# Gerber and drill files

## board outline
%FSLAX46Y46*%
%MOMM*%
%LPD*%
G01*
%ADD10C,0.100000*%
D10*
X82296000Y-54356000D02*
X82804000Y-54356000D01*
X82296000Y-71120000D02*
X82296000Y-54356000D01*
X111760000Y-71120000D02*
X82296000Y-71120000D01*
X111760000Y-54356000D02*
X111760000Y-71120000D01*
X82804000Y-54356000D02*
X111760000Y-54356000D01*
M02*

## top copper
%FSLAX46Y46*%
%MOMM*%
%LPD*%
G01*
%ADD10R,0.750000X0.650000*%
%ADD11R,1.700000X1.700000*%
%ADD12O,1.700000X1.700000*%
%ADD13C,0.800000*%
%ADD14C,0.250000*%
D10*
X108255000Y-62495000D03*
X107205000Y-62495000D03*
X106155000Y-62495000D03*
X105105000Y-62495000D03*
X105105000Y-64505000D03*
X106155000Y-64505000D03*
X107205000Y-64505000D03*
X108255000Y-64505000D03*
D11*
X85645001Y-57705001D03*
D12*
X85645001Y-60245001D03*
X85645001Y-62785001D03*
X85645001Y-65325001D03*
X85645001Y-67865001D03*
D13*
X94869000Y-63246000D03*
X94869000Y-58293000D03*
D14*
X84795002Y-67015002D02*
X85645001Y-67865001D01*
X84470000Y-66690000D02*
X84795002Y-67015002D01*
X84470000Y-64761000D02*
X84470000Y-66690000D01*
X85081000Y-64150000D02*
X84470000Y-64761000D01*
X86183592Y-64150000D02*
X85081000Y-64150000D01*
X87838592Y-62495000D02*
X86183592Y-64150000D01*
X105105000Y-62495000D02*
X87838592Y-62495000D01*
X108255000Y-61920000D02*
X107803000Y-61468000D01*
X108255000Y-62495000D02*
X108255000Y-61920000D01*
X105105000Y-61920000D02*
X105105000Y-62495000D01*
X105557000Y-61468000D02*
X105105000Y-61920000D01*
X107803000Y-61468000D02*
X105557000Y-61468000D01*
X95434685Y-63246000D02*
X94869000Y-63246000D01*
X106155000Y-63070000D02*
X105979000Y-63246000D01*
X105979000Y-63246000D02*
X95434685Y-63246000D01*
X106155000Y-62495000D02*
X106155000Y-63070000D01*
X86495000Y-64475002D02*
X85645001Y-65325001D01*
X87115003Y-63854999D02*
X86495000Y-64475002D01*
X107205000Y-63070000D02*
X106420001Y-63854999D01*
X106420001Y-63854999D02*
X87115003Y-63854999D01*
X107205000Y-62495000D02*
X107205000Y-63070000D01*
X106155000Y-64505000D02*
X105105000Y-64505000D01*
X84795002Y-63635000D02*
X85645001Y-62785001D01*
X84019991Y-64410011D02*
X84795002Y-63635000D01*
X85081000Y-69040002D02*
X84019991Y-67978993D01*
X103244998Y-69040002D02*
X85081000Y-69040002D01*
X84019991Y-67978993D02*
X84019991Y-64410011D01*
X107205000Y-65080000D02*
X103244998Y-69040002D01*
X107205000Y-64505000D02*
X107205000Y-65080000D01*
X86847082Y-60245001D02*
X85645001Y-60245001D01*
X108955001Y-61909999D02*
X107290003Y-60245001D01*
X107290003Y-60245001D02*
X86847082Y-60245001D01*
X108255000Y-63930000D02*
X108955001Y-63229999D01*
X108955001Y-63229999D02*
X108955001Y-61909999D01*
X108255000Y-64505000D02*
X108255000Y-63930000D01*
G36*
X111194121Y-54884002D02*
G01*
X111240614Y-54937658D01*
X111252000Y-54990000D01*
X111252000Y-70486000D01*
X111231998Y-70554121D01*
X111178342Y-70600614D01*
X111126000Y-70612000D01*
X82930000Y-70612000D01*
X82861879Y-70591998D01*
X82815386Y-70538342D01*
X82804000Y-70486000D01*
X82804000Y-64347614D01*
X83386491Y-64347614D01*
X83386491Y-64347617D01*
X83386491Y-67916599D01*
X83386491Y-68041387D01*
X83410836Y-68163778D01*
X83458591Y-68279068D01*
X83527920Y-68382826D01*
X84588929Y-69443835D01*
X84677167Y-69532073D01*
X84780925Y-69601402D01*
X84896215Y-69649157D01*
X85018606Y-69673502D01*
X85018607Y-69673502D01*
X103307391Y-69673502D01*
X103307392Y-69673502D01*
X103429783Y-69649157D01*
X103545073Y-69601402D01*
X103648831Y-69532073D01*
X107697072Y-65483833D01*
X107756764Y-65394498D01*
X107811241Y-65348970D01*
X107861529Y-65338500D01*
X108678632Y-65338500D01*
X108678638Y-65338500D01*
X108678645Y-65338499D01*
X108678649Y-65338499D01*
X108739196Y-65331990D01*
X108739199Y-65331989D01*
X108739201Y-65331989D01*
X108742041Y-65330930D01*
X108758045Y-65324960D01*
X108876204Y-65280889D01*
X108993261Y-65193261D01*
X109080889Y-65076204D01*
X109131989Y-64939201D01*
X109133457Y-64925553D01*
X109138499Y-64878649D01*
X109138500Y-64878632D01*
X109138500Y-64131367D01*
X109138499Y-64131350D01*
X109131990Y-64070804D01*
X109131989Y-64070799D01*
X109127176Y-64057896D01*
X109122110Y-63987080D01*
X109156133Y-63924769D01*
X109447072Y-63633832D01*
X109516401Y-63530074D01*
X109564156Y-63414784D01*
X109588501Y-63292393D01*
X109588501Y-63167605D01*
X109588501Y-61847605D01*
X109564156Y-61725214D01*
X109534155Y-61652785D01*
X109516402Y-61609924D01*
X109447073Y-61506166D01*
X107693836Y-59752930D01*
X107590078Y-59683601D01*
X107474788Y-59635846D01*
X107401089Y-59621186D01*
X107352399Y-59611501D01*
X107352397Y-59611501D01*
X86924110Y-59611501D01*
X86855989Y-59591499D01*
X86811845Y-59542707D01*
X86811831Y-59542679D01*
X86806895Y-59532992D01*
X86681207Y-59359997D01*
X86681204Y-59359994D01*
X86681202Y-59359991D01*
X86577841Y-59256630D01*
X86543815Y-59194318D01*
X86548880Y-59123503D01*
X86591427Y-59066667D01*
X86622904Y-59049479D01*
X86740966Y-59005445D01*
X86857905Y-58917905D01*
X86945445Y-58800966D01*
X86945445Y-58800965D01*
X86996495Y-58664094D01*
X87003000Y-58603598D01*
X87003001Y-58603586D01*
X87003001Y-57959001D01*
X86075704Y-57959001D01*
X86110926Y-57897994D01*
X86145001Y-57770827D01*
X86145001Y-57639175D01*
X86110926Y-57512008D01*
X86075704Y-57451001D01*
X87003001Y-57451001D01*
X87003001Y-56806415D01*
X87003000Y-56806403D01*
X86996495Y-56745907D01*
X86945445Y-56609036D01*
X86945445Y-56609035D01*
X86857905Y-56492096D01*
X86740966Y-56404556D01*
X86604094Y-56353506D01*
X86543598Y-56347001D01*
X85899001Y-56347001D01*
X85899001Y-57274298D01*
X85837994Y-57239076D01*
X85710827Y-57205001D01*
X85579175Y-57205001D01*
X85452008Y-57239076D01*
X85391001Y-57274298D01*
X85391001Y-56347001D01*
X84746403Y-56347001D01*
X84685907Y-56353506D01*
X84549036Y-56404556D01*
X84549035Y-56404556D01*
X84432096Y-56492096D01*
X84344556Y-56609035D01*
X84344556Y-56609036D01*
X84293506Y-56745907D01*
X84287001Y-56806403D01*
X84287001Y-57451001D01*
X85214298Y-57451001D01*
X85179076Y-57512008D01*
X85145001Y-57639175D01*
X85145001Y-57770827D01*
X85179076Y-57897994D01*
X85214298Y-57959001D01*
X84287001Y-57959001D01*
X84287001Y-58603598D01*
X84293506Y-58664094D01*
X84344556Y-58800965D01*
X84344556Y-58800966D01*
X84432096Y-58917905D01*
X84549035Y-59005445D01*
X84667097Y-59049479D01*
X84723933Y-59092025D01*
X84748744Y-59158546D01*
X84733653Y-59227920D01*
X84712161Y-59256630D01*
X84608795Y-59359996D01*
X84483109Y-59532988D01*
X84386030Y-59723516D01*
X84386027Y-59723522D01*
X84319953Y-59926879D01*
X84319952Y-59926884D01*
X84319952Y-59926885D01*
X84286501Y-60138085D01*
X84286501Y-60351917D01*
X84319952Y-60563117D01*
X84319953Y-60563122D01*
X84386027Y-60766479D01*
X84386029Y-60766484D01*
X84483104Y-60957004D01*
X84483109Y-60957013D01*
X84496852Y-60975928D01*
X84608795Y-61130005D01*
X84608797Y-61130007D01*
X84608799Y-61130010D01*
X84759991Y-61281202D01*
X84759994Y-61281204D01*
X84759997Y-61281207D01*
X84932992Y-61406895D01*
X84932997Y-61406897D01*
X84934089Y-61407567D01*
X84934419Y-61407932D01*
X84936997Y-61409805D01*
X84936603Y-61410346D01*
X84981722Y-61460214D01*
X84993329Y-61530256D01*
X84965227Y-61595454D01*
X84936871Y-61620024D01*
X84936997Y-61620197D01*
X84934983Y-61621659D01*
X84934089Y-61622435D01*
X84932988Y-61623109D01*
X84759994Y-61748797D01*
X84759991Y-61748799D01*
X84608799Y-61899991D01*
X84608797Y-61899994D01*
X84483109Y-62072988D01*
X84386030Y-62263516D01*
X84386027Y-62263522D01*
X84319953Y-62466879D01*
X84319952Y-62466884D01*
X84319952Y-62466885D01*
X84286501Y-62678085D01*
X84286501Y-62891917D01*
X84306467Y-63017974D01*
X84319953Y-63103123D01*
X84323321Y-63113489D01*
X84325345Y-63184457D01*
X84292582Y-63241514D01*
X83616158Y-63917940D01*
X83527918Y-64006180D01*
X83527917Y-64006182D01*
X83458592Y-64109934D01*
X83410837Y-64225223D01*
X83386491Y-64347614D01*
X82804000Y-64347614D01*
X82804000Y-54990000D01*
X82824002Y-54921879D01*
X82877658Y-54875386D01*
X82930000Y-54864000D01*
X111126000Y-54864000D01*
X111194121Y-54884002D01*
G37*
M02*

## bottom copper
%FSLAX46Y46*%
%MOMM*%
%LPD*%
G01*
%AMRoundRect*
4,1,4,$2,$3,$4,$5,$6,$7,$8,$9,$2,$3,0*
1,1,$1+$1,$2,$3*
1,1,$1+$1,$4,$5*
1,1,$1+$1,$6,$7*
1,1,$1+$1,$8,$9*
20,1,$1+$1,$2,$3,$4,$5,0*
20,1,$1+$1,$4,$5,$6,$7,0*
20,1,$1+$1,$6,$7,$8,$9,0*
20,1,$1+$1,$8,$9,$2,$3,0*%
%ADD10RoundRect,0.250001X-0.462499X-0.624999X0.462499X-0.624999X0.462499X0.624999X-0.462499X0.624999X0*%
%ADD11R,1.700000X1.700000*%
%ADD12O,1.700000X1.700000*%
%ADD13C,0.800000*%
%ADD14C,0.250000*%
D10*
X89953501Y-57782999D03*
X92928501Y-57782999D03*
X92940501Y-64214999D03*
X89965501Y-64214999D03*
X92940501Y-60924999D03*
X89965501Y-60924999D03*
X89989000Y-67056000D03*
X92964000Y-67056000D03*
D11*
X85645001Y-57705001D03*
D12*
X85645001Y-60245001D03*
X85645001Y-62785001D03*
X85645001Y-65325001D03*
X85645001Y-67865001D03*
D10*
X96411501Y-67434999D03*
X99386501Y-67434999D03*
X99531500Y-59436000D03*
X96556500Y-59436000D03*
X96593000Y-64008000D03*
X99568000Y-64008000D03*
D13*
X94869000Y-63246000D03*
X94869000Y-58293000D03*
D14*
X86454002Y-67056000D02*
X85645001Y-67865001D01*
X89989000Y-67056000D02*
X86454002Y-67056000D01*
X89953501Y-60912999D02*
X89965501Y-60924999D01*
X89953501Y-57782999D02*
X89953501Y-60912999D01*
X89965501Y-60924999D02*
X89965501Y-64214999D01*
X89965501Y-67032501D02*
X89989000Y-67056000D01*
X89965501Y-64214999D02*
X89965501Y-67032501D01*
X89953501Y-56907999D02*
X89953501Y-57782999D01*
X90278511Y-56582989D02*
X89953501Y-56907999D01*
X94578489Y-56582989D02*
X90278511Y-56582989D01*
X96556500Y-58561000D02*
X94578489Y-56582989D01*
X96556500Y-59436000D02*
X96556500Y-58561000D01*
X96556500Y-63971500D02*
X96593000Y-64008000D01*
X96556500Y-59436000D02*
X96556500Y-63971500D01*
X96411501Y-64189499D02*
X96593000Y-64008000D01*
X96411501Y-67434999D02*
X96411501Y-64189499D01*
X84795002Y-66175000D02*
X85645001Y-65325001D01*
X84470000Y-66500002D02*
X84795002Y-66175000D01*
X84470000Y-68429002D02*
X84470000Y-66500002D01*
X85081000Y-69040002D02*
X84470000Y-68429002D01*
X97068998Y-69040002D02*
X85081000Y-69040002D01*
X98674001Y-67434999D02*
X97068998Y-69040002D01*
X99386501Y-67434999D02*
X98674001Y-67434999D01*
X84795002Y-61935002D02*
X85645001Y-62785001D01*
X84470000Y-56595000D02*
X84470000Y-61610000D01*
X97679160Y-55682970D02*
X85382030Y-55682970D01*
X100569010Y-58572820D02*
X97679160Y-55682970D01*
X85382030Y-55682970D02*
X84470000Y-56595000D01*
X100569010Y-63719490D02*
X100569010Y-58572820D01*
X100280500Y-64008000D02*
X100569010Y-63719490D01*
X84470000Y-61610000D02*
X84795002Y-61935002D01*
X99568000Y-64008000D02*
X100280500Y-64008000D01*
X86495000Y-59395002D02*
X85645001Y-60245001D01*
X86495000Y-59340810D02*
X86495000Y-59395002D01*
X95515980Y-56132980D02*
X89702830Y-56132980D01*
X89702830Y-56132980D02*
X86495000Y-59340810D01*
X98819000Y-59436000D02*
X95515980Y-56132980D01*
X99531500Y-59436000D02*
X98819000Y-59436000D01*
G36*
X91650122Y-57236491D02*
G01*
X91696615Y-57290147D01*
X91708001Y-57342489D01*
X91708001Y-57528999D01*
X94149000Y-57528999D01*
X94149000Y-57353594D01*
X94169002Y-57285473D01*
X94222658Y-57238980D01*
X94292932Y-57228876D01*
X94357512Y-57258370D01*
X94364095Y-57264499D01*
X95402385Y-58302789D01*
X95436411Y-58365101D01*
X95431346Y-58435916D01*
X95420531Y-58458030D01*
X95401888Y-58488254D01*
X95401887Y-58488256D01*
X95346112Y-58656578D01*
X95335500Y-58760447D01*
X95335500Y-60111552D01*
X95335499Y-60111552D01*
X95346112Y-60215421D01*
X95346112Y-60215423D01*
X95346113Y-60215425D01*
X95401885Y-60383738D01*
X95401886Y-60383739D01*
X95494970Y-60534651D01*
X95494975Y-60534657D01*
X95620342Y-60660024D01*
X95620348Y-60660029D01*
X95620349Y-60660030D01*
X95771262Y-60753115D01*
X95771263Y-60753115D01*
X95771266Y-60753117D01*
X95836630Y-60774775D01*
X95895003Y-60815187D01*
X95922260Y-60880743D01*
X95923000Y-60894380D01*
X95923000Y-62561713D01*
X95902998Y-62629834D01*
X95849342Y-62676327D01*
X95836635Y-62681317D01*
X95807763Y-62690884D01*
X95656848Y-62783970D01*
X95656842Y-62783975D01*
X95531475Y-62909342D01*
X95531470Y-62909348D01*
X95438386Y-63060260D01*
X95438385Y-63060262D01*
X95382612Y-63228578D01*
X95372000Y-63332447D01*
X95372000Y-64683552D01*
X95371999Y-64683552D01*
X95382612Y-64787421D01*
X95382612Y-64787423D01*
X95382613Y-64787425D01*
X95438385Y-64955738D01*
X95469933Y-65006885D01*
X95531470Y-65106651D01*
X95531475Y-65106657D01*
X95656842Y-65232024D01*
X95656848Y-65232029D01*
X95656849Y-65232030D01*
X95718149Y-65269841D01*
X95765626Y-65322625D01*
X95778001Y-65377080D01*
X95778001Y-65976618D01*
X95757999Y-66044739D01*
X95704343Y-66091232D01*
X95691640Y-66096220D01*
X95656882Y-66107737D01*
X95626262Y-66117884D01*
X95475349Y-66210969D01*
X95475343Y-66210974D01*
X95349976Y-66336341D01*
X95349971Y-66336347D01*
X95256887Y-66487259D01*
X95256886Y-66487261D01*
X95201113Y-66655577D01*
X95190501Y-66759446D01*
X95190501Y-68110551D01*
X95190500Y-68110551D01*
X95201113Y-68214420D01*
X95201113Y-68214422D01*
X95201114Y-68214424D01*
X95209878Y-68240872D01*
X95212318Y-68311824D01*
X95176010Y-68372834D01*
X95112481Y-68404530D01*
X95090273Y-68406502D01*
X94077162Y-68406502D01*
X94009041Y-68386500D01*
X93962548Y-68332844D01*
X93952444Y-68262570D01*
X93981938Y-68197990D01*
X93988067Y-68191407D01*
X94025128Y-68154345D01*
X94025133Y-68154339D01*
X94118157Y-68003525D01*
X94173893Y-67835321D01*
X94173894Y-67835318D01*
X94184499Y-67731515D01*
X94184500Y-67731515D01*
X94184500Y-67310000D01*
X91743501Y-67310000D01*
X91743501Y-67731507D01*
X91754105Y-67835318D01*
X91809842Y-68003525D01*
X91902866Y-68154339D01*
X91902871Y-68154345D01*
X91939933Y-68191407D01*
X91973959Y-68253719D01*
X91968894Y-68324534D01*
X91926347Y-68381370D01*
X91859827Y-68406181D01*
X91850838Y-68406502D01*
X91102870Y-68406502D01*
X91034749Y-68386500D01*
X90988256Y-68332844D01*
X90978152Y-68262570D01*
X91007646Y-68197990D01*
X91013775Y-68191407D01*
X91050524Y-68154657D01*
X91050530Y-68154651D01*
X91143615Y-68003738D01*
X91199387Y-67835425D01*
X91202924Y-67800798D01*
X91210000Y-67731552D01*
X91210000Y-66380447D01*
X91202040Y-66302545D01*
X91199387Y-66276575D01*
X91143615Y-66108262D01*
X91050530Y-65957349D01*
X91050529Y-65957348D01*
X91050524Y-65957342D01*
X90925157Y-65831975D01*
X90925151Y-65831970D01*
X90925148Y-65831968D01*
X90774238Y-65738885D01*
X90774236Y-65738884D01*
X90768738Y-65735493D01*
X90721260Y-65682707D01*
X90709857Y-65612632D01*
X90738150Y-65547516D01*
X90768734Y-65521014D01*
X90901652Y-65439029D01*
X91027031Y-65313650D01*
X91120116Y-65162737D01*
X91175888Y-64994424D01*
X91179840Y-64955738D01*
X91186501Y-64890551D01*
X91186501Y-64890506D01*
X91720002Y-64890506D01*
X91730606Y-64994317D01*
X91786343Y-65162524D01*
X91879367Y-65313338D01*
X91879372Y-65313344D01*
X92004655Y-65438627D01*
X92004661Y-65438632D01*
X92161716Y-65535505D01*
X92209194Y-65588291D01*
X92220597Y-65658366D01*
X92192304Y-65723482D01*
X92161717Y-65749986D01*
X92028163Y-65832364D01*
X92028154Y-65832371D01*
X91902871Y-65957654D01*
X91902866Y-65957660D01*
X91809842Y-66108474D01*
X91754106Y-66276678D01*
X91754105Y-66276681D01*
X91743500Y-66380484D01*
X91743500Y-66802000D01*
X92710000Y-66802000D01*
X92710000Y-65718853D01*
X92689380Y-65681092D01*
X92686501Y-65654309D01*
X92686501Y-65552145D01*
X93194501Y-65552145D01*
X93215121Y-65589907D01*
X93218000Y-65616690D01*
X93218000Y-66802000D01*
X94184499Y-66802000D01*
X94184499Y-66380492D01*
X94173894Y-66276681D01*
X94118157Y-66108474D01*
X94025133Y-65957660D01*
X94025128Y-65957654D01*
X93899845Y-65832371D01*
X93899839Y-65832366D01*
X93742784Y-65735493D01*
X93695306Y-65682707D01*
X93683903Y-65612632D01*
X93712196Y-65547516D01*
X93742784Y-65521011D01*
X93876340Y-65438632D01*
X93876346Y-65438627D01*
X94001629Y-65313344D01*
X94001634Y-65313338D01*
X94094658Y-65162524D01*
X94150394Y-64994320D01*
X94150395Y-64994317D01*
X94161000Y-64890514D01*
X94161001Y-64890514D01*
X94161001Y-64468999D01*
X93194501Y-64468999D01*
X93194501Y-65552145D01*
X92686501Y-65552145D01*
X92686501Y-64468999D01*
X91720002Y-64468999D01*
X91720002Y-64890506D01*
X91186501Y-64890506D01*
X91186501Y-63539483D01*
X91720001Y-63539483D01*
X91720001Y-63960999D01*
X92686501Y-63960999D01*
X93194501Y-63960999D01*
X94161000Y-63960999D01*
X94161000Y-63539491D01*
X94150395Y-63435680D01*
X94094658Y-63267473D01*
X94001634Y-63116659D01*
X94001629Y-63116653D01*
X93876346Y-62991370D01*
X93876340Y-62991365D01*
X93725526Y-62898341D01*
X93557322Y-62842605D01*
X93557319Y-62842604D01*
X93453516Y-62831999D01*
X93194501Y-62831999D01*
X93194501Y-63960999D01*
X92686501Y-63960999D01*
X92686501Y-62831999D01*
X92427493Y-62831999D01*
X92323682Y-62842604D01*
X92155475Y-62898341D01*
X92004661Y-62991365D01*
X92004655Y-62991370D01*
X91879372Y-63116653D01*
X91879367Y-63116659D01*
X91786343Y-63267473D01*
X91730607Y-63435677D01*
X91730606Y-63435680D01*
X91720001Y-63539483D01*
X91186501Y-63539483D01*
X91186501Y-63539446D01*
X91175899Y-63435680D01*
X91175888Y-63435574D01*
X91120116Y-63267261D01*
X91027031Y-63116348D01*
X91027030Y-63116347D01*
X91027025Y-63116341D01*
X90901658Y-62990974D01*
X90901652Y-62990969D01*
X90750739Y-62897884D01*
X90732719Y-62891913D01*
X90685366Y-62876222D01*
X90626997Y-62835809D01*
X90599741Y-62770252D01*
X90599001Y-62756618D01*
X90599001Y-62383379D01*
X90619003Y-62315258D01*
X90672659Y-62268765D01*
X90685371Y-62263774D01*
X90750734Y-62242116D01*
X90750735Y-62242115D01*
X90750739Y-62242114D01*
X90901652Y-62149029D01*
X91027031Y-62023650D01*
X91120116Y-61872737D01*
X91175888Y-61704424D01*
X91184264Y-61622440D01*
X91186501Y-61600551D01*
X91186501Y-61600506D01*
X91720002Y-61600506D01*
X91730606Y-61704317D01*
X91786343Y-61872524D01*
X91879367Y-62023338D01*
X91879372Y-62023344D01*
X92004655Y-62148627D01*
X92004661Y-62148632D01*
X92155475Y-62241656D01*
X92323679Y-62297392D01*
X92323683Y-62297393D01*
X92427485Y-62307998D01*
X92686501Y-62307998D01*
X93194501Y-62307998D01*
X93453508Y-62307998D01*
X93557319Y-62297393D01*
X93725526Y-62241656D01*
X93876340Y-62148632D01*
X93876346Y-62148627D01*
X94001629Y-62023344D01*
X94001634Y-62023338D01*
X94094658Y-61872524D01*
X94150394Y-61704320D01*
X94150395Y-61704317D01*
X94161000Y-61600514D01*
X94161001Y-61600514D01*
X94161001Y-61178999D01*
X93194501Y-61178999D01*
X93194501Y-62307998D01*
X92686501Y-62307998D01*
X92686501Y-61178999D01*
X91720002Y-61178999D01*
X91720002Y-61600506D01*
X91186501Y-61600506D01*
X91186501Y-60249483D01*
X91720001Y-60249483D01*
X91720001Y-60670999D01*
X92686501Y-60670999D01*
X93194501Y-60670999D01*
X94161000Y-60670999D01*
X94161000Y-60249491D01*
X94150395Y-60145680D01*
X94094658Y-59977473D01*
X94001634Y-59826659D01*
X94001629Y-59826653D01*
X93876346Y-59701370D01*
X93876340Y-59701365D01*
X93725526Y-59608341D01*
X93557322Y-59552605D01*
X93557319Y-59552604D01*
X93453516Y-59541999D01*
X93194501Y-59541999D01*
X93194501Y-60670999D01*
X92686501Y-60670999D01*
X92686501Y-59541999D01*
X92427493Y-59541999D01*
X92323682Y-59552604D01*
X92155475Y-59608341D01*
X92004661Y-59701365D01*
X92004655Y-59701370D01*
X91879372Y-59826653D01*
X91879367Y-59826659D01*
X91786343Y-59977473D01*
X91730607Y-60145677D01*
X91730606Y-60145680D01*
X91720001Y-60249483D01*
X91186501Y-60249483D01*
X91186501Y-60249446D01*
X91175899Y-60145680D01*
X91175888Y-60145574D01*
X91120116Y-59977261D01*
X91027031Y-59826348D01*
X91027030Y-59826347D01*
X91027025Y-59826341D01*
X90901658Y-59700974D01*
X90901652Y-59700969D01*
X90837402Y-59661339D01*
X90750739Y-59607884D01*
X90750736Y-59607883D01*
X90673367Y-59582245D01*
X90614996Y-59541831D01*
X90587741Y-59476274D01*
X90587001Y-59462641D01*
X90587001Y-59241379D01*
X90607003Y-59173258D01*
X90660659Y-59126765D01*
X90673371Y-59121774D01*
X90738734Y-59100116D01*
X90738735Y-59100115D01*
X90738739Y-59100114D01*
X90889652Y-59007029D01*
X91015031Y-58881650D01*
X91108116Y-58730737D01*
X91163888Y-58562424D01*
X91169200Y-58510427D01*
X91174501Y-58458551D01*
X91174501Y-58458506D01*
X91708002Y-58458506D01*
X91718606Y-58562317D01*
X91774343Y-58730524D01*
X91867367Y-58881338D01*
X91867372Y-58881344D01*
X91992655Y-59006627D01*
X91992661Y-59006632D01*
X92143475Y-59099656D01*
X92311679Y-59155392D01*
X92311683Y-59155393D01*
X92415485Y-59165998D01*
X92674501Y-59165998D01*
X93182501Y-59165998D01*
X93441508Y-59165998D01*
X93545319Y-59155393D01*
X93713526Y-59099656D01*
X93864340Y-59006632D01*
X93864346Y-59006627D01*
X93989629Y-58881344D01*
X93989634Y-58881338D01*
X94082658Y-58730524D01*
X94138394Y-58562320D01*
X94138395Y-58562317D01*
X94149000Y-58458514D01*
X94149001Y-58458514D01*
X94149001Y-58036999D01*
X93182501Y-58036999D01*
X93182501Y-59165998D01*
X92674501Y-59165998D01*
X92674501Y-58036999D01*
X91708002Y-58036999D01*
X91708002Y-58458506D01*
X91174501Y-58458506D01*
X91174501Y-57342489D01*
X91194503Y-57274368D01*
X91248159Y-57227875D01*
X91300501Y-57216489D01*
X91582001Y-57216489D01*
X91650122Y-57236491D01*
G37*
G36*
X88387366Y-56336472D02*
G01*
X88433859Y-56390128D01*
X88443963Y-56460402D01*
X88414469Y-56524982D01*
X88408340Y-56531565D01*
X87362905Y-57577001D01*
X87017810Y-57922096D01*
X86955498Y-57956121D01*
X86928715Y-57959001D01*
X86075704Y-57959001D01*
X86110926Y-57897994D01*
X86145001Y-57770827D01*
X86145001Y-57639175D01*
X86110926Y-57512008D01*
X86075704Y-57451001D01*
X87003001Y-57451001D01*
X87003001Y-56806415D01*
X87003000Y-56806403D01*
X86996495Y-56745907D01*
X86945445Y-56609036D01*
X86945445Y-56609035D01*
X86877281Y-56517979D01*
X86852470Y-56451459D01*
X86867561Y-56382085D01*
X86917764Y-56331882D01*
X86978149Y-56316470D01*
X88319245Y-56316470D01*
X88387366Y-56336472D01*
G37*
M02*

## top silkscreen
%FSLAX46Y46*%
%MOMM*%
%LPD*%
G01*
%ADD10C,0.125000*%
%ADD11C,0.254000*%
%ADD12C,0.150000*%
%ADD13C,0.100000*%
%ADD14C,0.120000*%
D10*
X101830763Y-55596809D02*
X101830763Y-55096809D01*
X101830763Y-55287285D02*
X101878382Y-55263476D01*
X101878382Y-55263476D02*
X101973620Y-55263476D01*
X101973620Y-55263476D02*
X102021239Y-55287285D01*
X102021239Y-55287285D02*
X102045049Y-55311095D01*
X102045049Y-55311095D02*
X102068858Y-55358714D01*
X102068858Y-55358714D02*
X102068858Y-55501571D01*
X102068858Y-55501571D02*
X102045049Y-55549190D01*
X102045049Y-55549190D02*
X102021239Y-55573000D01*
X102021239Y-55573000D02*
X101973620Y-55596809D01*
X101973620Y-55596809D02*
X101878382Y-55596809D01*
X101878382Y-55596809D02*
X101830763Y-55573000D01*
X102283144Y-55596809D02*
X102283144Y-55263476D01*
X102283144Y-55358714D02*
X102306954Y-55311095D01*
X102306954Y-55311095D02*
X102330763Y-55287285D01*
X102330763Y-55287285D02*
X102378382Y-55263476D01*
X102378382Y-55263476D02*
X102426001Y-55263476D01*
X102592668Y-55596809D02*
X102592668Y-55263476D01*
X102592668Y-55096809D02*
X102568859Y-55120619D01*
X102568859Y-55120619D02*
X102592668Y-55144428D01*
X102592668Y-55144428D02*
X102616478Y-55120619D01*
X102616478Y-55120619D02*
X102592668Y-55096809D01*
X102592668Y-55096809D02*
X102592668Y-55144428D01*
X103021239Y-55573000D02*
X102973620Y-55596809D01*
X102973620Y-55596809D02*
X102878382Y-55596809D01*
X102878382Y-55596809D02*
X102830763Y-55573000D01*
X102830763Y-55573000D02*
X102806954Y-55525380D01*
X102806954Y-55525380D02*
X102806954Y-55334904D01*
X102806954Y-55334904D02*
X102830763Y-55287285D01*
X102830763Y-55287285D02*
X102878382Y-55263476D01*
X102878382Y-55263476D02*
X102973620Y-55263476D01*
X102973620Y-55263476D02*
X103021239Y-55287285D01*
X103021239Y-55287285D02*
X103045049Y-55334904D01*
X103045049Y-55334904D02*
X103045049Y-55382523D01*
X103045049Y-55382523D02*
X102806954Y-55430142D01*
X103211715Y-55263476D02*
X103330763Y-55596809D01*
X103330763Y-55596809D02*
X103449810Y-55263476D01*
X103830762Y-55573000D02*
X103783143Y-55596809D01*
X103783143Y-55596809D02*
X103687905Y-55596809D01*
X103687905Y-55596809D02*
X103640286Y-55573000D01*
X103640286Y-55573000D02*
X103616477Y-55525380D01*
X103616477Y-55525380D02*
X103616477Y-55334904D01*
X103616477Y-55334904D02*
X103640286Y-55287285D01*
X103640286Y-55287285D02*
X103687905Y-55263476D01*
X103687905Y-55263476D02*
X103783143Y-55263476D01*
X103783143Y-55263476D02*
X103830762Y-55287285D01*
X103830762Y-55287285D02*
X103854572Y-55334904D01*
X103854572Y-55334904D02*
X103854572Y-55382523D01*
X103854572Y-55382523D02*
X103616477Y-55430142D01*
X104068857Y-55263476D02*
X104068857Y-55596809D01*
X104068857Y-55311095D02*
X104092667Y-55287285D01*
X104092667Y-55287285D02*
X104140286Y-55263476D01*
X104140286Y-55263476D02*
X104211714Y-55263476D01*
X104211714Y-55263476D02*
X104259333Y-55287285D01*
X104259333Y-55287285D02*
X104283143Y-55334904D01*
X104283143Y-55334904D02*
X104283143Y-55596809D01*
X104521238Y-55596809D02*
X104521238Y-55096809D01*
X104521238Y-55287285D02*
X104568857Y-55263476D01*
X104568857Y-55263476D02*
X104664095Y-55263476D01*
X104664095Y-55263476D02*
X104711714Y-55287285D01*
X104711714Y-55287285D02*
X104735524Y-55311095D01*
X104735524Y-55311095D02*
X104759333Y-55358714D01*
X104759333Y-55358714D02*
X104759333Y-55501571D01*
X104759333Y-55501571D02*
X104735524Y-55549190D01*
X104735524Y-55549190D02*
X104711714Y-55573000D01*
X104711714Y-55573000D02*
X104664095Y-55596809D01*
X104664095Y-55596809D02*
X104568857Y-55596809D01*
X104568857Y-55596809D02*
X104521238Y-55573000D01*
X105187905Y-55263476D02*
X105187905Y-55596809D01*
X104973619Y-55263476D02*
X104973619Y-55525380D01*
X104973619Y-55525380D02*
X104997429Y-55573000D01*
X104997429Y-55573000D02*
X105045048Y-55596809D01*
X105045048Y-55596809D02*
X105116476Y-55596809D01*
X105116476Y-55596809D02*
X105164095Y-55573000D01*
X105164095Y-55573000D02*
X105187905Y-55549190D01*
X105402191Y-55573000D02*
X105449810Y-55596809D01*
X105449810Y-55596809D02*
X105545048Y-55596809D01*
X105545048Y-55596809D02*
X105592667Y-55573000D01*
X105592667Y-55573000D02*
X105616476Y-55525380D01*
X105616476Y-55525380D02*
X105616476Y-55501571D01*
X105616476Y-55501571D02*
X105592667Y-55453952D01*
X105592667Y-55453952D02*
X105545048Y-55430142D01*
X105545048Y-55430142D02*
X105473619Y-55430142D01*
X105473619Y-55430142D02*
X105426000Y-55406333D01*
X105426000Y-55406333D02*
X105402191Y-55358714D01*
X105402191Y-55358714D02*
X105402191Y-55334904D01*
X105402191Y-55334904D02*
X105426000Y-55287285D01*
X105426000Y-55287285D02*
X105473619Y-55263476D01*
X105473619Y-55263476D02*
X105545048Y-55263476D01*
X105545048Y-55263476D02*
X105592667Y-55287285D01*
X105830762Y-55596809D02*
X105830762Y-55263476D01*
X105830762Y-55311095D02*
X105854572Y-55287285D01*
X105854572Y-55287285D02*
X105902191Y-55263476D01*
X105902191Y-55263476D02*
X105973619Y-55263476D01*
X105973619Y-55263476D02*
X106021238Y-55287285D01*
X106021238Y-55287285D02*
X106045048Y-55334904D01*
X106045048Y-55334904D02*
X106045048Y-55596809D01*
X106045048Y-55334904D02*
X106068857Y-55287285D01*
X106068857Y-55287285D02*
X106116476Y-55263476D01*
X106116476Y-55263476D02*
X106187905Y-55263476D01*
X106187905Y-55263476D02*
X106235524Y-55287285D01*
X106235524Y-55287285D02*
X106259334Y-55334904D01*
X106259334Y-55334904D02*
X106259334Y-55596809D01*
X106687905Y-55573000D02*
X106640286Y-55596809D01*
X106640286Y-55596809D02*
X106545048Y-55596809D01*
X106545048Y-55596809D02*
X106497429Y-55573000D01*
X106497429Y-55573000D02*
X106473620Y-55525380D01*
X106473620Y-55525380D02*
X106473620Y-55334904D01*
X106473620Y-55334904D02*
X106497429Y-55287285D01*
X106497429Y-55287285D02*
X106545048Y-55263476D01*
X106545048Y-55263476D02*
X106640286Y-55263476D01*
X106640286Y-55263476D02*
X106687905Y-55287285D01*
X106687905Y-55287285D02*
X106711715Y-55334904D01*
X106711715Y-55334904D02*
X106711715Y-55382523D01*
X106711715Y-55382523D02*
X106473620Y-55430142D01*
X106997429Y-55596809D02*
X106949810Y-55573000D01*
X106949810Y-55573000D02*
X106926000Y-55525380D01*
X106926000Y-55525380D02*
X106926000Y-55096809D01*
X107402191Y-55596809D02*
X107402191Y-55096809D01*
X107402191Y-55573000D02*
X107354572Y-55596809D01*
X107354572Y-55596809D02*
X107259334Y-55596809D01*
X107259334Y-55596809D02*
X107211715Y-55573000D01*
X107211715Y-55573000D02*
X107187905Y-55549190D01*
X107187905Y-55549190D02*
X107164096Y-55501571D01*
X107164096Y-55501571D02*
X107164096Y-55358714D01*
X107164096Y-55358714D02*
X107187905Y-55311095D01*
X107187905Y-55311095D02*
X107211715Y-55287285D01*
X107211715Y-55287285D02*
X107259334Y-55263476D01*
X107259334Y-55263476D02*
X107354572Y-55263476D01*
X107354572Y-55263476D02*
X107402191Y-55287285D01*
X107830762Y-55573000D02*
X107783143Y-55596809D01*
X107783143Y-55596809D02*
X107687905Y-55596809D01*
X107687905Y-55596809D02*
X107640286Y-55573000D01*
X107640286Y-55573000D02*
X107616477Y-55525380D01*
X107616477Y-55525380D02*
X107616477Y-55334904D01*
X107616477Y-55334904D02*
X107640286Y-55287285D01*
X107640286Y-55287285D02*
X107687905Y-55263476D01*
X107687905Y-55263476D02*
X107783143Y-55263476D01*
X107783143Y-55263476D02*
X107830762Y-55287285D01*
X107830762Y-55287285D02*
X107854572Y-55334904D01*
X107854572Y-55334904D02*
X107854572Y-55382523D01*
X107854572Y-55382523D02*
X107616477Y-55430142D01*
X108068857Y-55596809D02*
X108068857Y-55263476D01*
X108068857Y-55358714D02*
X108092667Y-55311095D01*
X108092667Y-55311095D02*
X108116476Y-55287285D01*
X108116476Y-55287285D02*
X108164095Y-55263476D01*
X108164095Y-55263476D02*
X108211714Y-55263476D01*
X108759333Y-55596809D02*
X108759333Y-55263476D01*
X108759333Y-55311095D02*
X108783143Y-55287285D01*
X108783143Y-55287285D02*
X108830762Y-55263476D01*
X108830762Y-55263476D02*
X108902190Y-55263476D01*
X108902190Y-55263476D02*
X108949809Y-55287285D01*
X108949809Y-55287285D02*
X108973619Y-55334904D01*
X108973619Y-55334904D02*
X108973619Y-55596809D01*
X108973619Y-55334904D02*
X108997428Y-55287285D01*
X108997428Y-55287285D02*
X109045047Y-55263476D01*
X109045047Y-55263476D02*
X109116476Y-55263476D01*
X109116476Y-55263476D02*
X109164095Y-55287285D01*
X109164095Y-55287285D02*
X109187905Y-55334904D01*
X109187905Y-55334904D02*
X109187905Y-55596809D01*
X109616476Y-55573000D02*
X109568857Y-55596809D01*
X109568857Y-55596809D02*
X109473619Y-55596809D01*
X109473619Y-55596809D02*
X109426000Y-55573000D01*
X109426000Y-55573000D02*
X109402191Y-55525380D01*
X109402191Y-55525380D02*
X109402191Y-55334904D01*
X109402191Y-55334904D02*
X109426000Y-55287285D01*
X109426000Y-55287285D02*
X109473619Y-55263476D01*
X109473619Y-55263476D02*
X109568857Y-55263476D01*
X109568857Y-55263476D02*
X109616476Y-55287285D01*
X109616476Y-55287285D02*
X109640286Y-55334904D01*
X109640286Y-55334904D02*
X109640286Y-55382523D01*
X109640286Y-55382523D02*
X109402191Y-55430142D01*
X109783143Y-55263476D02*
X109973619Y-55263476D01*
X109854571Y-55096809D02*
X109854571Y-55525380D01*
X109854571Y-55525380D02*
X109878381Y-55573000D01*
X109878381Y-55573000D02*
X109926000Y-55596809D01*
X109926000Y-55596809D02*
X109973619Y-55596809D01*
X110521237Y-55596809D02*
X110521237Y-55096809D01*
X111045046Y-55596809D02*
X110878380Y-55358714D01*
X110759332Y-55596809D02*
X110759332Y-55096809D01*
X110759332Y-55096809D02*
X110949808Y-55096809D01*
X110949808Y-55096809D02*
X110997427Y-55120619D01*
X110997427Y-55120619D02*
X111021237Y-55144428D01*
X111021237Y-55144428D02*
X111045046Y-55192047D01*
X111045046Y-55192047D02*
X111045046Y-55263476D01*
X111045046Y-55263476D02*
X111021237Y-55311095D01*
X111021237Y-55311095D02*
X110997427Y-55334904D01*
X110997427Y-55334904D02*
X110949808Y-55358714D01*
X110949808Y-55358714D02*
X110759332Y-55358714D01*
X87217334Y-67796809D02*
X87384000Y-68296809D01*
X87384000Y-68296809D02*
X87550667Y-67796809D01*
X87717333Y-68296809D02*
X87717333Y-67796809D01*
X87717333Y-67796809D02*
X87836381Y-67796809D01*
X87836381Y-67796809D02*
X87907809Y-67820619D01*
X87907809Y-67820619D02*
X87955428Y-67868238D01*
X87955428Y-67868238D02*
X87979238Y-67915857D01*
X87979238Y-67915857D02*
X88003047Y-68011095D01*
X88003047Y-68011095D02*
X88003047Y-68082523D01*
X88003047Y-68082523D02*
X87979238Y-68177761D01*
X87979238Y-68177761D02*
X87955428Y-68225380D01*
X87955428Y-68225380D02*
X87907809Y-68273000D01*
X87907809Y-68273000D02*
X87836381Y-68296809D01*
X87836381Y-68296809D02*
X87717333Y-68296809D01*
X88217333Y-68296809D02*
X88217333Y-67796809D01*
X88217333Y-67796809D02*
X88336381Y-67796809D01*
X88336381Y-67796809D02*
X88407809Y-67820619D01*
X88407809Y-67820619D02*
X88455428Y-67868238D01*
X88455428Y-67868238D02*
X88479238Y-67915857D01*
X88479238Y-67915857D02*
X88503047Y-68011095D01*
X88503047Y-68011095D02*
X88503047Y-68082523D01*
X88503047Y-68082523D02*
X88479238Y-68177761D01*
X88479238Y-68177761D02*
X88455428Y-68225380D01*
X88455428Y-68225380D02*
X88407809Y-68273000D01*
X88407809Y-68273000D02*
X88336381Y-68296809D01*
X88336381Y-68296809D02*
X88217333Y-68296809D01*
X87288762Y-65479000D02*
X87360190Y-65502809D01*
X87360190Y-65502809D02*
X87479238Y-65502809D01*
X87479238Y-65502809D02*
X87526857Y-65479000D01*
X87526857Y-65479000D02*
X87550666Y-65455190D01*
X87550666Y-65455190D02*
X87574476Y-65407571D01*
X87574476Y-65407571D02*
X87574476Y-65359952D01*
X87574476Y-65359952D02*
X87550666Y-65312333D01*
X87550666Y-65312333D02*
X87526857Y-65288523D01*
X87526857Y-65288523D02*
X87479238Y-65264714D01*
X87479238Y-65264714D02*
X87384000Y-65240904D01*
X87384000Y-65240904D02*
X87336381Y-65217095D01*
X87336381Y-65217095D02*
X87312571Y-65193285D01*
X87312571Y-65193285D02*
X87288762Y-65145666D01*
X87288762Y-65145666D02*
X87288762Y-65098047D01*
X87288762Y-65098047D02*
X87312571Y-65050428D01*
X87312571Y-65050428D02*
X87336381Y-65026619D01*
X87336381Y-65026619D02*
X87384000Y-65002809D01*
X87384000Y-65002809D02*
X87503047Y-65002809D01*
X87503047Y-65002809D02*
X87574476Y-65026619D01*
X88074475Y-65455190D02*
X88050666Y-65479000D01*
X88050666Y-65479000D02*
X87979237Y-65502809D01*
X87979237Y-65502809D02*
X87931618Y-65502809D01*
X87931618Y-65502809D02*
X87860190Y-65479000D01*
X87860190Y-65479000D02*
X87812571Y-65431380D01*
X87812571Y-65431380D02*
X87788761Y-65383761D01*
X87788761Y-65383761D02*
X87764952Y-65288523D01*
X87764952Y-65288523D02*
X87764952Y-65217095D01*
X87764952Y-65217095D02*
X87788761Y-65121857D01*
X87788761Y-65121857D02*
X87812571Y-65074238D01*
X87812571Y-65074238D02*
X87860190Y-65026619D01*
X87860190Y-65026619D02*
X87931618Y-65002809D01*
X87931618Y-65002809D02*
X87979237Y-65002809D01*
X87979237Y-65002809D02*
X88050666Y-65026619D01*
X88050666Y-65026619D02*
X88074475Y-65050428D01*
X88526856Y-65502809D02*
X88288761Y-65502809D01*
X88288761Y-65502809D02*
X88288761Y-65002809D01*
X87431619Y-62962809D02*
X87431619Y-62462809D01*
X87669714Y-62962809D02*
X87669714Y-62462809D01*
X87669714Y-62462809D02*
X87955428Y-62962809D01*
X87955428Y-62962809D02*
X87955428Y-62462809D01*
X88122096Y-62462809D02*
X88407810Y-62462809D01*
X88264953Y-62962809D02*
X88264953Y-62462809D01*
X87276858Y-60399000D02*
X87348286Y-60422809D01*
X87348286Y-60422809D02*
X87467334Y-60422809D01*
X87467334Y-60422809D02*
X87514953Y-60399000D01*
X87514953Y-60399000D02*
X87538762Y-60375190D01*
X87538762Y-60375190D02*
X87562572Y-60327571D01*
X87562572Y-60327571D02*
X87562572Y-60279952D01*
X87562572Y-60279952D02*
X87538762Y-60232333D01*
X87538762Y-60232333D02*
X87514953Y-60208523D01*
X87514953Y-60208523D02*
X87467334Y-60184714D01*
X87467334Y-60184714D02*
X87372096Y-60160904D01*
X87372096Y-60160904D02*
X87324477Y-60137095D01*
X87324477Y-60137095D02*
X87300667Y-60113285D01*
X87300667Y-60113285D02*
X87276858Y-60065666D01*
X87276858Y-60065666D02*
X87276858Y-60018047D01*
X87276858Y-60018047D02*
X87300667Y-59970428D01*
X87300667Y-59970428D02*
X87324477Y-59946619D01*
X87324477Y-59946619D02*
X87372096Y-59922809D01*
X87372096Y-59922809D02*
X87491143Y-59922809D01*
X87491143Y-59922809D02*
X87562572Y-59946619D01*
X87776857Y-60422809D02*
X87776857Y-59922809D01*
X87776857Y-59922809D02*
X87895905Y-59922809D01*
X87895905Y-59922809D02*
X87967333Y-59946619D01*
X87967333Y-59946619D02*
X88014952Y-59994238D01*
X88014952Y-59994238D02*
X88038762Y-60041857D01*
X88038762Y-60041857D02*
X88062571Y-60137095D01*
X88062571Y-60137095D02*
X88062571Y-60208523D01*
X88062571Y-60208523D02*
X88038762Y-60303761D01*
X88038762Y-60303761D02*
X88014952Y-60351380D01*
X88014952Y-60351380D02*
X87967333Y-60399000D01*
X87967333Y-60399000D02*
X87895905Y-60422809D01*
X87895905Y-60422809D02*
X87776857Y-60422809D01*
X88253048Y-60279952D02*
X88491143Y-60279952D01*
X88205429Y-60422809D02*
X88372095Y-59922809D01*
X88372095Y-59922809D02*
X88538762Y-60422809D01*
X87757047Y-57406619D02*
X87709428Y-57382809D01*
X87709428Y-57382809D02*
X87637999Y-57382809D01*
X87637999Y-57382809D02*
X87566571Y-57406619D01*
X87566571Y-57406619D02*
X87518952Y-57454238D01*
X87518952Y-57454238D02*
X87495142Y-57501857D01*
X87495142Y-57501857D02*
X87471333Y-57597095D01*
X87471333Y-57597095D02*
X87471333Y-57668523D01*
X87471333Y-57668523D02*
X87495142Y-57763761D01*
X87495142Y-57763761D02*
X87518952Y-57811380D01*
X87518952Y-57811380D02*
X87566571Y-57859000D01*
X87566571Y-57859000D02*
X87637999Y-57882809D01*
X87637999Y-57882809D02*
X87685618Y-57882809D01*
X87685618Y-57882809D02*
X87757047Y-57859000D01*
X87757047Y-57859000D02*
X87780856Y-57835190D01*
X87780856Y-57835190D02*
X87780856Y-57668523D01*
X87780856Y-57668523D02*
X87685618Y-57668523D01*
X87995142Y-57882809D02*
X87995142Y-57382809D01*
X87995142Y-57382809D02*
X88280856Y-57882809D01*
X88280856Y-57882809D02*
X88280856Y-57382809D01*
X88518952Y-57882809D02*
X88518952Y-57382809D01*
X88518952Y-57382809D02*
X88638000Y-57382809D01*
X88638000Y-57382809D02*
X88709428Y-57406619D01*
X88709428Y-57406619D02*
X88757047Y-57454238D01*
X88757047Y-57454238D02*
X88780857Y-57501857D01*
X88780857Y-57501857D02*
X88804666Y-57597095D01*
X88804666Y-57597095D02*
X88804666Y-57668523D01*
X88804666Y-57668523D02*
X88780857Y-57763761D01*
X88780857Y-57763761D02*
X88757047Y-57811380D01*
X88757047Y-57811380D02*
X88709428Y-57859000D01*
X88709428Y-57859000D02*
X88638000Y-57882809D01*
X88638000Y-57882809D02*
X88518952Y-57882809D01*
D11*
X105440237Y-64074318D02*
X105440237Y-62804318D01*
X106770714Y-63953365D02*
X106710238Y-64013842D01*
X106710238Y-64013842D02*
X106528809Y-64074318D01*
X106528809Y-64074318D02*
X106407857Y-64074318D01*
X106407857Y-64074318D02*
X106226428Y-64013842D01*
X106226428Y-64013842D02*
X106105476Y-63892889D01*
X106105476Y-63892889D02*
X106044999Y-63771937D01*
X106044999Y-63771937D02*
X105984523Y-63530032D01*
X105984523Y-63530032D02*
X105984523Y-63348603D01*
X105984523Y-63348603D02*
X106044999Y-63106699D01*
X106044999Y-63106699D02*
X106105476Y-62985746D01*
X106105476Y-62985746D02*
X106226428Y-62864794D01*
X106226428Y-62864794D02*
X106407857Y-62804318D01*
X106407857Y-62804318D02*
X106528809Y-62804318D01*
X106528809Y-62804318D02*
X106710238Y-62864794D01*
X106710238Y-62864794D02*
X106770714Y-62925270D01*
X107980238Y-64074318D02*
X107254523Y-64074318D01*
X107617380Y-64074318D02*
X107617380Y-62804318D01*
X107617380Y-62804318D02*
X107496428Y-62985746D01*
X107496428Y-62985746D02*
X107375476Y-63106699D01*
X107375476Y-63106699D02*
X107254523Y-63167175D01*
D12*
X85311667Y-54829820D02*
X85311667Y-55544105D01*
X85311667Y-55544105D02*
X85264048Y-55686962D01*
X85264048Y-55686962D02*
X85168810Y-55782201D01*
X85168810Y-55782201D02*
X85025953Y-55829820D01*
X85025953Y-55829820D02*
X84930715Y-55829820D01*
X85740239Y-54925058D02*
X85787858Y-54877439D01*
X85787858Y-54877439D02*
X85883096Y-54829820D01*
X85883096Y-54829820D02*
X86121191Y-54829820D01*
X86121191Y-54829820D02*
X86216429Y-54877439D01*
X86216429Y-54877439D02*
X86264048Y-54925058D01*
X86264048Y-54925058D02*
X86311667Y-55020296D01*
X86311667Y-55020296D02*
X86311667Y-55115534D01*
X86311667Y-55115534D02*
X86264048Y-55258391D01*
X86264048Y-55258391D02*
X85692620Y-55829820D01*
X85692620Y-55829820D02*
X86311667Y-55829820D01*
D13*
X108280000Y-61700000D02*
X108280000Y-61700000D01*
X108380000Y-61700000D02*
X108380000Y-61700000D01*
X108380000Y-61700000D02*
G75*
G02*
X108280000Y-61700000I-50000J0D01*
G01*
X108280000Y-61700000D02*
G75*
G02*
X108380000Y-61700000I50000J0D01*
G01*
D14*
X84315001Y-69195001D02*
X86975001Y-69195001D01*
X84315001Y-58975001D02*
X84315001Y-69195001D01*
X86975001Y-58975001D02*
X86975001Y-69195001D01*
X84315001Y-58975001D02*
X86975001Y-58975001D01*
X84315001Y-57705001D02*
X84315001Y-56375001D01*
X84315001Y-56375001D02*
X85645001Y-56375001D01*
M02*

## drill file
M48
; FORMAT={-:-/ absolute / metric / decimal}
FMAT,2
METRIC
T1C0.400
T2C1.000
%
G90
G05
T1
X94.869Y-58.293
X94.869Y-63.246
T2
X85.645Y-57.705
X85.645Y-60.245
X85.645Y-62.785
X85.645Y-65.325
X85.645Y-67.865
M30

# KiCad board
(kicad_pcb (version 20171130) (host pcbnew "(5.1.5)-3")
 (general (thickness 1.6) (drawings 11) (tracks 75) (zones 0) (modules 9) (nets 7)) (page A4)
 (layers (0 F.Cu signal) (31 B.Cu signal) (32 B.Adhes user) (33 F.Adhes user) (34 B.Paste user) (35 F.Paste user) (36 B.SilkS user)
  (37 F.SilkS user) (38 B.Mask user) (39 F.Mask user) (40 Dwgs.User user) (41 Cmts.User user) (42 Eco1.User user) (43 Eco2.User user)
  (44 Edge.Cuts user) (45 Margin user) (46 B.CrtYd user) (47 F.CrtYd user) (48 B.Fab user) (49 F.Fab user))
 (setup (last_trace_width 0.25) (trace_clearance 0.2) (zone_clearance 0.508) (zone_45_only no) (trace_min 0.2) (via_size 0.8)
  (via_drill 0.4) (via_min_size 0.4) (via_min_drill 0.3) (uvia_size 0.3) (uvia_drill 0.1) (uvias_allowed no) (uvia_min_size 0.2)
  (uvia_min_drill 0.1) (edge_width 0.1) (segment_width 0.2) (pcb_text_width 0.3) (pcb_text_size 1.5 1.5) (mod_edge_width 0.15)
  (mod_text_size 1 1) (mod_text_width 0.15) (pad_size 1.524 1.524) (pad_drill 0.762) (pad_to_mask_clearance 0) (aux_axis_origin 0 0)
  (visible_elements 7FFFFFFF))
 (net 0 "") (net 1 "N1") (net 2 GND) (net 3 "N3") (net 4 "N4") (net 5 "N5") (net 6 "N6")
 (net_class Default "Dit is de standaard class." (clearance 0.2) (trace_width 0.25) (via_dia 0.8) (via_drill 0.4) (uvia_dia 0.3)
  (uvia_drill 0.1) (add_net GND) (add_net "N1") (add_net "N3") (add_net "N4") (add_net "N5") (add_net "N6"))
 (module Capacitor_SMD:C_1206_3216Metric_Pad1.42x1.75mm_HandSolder (layer B.Cu) (at 91.441001 57.782999)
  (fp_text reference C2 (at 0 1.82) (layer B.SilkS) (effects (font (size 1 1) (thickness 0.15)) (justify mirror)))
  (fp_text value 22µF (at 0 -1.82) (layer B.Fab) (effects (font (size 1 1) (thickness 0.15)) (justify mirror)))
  (pad 1 smd roundrect (at -1.4875 0) (size 1.425 1.75) (layers B.Cu B.Paste B.Mask) (roundrect_rratio 0.175439) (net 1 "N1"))
  (pad 2 smd roundrect (at 1.4875 0) (size 1.425 1.75) (layers B.Cu B.Paste B.Mask) (roundrect_rratio 0.175439) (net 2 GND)))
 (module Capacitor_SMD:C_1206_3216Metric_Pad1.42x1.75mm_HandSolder (layer B.Cu) (at 91.453001 64.214999)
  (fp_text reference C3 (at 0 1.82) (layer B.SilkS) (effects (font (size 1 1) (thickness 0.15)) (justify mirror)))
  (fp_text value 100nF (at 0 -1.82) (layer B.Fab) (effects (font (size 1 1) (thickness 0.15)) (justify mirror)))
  (pad 2 smd roundrect (at 1.4875 0) (size 1.425 1.75) (layers B.Cu B.Paste B.Mask) (roundrect_rratio 0.175439) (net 2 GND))
  (pad 1 smd roundrect (at -1.4875 0) (size 1.425 1.75) (layers B.Cu B.Paste B.Mask) (roundrect_rratio 0.175439) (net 1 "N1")))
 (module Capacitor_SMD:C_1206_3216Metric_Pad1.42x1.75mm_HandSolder (layer B.Cu) (at 91.453001 60.924999)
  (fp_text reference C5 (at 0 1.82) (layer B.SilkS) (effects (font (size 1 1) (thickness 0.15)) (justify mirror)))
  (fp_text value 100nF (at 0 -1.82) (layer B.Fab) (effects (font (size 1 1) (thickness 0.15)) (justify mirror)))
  (pad 2 smd roundrect (at 1.4875 0) (size 1.425 1.75) (layers B.Cu B.Paste B.Mask) (roundrect_rratio 0.175439) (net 2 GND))
  (pad 1 smd roundrect (at -1.4875 0) (size 1.425 1.75) (layers B.Cu B.Paste B.Mask) (roundrect_rratio 0.175439) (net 1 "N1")))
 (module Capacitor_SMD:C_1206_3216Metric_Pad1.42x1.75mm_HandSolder (layer B.Cu) (at 91.4765 67.056)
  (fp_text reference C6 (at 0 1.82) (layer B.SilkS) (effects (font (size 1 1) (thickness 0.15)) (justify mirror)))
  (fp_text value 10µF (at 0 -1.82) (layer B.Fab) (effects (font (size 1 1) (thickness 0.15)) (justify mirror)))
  (pad 1 smd roundrect (at -1.4875 0) (size 1.425 1.75) (layers B.Cu B.Paste B.Mask) (roundrect_rratio 0.175439) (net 1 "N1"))
  (pad 2 smd roundrect (at 1.4875 0) (size 1.425 1.75) (layers B.Cu B.Paste B.Mask) (roundrect_rratio 0.175439) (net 2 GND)))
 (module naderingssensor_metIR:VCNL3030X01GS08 (layer F.Cu) (at 106.68 63.5)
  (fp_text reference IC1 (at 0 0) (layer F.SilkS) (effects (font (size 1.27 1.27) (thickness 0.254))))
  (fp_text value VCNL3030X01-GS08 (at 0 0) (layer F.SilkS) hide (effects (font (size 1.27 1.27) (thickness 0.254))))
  (fp_line (start 1.6 -1.8) (end 1.6 -1.8) (layer F.SilkS) (width 0.1))
  (fp_line (start 1.7 -1.8) (end 1.7 -1.8) (layer F.SilkS) (width 0.1))
  (fp_arc (start 1.65 -1.8) (end 1.6 -1.8) (angle -180) (layer F.SilkS) (width 0.1))
  (fp_arc (start 1.65 -1.8) (end 1.7 -1.8) (angle -180) (layer F.SilkS) (width 0.1))
  (pad 1 smd rect (at 1.575 -1.005 90) (size 0.65 0.75) (layers F.Cu F.Paste F.Mask) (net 1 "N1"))
  (pad 2 smd rect (at 0.525 -1.005 90) (size 0.65 0.75) (layers F.Cu F.Paste F.Mask) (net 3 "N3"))
  (pad 3 smd rect (at -0.525 -1.005 90) (size 0.65 0.75) (layers F.Cu F.Paste F.Mask) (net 2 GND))
  (pad 4 smd rect (at -1.575 -1.005 90) (size 0.65 0.75) (layers F.Cu F.Paste F.Mask) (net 1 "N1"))
  (pad 5 smd rect (at -1.575 1.005 90) (size 0.65 0.75) (layers F.Cu F.Paste F.Mask) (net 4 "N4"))
  (pad 6 smd rect (at -0.525 1.005 90) (size 0.65 0.75) (layers F.Cu F.Paste F.Mask) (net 4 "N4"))
  (pad 7 smd rect (at 0.525 1.005 90) (size 0.65 0.75) (layers F.Cu F.Paste F.Mask) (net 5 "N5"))
  (pad 8 smd rect (at 1.575 1.005 90) (size 0.65 0.75) (layers F.Cu F.Paste F.Mask) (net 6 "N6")))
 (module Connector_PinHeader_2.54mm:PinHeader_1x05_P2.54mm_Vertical (layer F.Cu) (at 85.645001 57.705001)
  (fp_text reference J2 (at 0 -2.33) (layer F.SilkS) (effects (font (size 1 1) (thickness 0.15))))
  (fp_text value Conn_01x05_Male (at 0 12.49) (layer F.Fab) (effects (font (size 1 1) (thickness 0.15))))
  (fp_line (start -1.33 11.49) (end 1.33 11.49) (layer F.SilkS) (width 0.12))
  (fp_line (start -1.33 1.27) (end -1.33 11.49) (layer F.SilkS) (width 0.12))
  (fp_line (start 1.33 1.27) (end 1.33 11.49) (layer F.SilkS) (width 0.12))
  (fp_line (start -1.33 1.27) (end 1.33 1.27) (layer F.SilkS) (width 0.12))
  (fp_line (start -1.33 0) (end -1.33 -1.33) (layer F.SilkS) (width 0.12))
  (fp_line (start -1.33 -1.33) (end 0 -1.33) (layer F.SilkS) (width 0.12))
  (pad 1 thru_hole rect (at 0 0) (size 1.7 1.7) (drill 1) (layers *.Cu *.Mask) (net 2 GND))
  (pad 2 thru_hole oval (at 0 2.54) (size 1.7 1.7) (drill 1) (layers *.Cu *.Mask) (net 6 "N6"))
  (pad 3 thru_hole oval (at 0 5.08) (size 1.7 1.7) (drill 1) (layers *.Cu *.Mask) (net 5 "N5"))
  (pad 4 thru_hole oval (at 0 7.62) (size 1.7 1.7) (drill 1) (layers *.Cu *.Mask) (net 3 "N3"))
  (pad 5 thru_hole oval (at 0 10.16) (size 1.7 1.7) (drill 1) (layers *.Cu *.Mask) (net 1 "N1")))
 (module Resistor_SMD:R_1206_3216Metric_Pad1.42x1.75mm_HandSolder (layer B.Cu) (at 97.899001 67.434999)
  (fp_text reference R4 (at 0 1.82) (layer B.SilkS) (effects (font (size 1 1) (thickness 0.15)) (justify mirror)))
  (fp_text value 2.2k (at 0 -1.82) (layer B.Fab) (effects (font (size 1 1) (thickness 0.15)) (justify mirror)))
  (pad 1 smd roundrect (at -1.4875 0) (size 1.425 1.75) (layers B.Cu B.Paste B.Mask) (roundrect_rratio 0.175439) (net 1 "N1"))
  (pad 2 smd roundrect (at 1.4875 0) (size 1.425 1.75) (layers B.Cu B.Paste B.Mask) (roundrect_rratio 0.175439) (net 3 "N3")))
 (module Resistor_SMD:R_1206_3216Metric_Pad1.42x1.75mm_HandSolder (layer B.Cu) (at 98.044 59.436)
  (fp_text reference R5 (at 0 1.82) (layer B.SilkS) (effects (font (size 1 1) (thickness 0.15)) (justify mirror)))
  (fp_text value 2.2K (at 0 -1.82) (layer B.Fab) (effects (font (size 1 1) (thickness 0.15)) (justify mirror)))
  (pad 2 smd roundrect (at 1.4875 0) (size 1.425 1.75) (layers B.Cu B.Paste B.Mask) (roundrect_rratio 0.175439) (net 6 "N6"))
  (pad 1 smd roundrect (at -1.4875 0) (size 1.425 1.75) (layers B.Cu B.Paste B.Mask) (roundrect_rratio 0.175439) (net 1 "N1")))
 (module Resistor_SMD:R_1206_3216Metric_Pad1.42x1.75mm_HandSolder (layer B.Cu) (at 98.0805 64.008)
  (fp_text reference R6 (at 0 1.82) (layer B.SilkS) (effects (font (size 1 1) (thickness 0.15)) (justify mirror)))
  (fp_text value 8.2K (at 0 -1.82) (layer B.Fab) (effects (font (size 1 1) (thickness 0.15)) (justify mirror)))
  (pad 1 smd roundrect (at -1.4875 0) (size 1.425 1.75) (layers B.Cu B.Paste B.Mask) (roundrect_rratio 0.175439) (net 1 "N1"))
  (pad 2 smd roundrect (at 1.4875 0) (size 1.425 1.75) (layers B.Cu B.Paste B.Mask) (roundrect_rratio 0.175439) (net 5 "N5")))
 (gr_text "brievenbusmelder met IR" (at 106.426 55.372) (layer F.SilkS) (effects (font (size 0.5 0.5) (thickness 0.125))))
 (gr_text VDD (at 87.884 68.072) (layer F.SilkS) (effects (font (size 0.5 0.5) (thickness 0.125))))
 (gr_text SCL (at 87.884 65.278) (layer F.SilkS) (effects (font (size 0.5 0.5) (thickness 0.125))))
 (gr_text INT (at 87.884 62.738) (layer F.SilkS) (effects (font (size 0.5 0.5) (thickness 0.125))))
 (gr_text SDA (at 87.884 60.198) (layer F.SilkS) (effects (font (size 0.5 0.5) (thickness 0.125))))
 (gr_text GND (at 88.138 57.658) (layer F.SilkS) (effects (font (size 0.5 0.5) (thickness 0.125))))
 (gr_line (start 82.296 54.356) (end 82.804 54.356) (layer Edge.Cuts) (width 0.1))
 (gr_line (start 82.296 71.12) (end 82.296 54.356) (layer Edge.Cuts) (width 0.1))
 (gr_line (start 111.76 71.12) (end 82.296 71.12) (layer Edge.Cuts) (width 0.1))
 (gr_line (start 111.76 54.356) (end 111.76 71.12) (layer Edge.Cuts) (width 0.1))
 (gr_line (start 82.804 54.356) (end 111.76 54.356) (layer Edge.Cuts) (width 0.1))
 (segment (start 86.454002 67.056) (end 85.645001 67.865001) (width 0.25) (layer B.Cu) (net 1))
 (segment (start 89.989 67.056) (end 86.454002 67.056) (width 0.25) (layer B.Cu) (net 1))
 (segment (start 89.953501 60.912999) (end 89.965501 60.924999) (width 0.25) (layer B.Cu) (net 1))
 (segment (start 89.953501 57.782999) (end 89.953501 60.912999) (width 0.25) (layer B.Cu) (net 1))
 (segment (start 89.965501 60.924999) (end 89.965501 64.214999) (width 0.25) (layer B.Cu) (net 1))
 (segment (start 89.965501 67.032501) (end 89.989 67.056) (width 0.25) (layer B.Cu) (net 1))
 (segment (start 89.965501 64.214999) (end 89.965501 67.032501) (width 0.25) (layer B.Cu) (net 1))
 (segment (start 89.953501 56.907999) (end 89.953501 57.782999) (width 0.25) (layer B.Cu) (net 1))
 (segment (start 90.278511 56.582989) (end 89.953501 56.907999) (width 0.25) (layer B.Cu) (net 1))
 (segment (start 94.578489 56.582989) (end 90.278511 56.582989) (width 0.25) (layer B.Cu) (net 1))
 (segment (start 96.5565 58.561) (end 94.578489 56.582989) (width 0.25) (layer B.Cu) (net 1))
 (segment (start 96.5565 59.436) (end 96.5565 58.561) (width 0.25) (layer B.Cu) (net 1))
 (segment (start 96.5565 63.9715) (end 96.593 64.008) (width 0.25) (layer B.Cu) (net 1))
 (segment (start 96.5565 59.436) (end 96.5565 63.9715) (width 0.25) (layer B.Cu) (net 1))
 (segment (start 96.411501 64.189499) (end 96.593 64.008) (width 0.25) (layer B.Cu) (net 1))
 (segment (start 96.411501 67.434999) (end 96.411501 64.189499) (width 0.25) (layer B.Cu) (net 1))
 (segment (start 84.795002 67.015002) (end 85.645001 67.865001) (width 0.25) (layer F.Cu) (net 1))
 (segment (start 84.47 66.69) (end 84.795002 67.015002) (width 0.25) (layer F.Cu) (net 1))
 (segment (start 84.47 64.761) (end 84.47 66.69) (width 0.25) (layer F.Cu) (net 1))
 (segment (start 85.081 64.15) (end 84.47 64.761) (width 0.25) (layer F.Cu) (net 1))
 (segment (start 86.183592 64.15) (end 85.081 64.15) (width 0.25) (layer F.Cu) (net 1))
 (segment (start 87.838592 62.495) (end 86.183592 64.15) (width 0.25) (layer F.Cu) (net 1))
 (segment (start 105.105 62.495) (end 87.838592 62.495) (width 0.25) (layer F.Cu) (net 1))
 (segment (start 108.255 61.92) (end 107.803 61.468) (width 0.25) (layer F.Cu) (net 1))
 (segment (start 108.255 62.495) (end 108.255 61.92) (width 0.25) (layer F.Cu) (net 1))
 (segment (start 105.105 61.92) (end 105.105 62.495) (width 0.25) (layer F.Cu) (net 1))
 (segment (start 105.557 61.468) (end 105.105 61.92) (width 0.25) (layer F.Cu) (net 1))
 (segment (start 107.803 61.468) (end 105.557 61.468) (width 0.25) (layer F.Cu) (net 1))
 (via (at 94.869 63.246) (size 0.8) (drill 0.4) (layers F.Cu B.Cu) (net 2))
 (segment (start 95.434685 63.246) (end 94.869 63.246) (width 0.25) (layer F.Cu) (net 2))
 (segment (start 106.155 63.07) (end 105.979 63.246) (width 0.25) (layer F.Cu) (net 2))
 (segment (start 105.979 63.246) (end 95.434685 63.246) (width 0.25) (layer F.Cu) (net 2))
 (segment (start 106.155 62.495) (end 106.155 63.07) (width 0.25) (layer F.Cu) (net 2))
 (via (at 94.869 58.293) (size 0.8) (drill 0.4) (layers F.Cu B.Cu) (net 2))
 (segment (start 84.795002 66.175) (end 85.645001 65.325001) (width 0.25) (layer B.Cu) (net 3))
 (segment (start 84.47 66.500002) (end 84.795002 66.175) (width 0.25) (layer B.Cu) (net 3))
 (segment (start 84.47 68.429002) (end 84.47 66.500002) (width 0.25) (layer B.Cu) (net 3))
 (segment (start 85.081 69.040002) (end 84.47 68.429002) (width 0.25) (layer B.Cu) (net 3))
 (segment (start 97.068998 69.040002) (end 85.081 69.040002) (width 0.25) (layer B.Cu) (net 3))
 (segment (start 98.674001 67.434999) (end 97.068998 69.040002) (width 0.25) (layer B.Cu) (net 3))
 (segment (start 99.386501 67.434999) (end 98.674001 67.434999) (width 0.25) (layer B.Cu) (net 3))
 (segment (start 86.495 64.475002) (end 85.645001 65.325001) (width 0.25) (layer F.Cu) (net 3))
 (segment (start 87.115003 63.854999) (end 86.495 64.475002) (width 0.25) (layer F.Cu) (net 3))
 (segment (start 107.205 63.07) (end 106.420001 63.854999) (width 0.25) (layer F.Cu) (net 3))
 (segment (start 106.420001 63.854999) (end 87.115003 63.854999) (width 0.25) (layer F.Cu) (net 3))
 (segment (start 107.205 62.495) (end 107.205 63.07) (width 0.25) (layer F.Cu) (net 3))
 (segment (start 106.155 64.505) (end 105.105 64.505) (width 0.25) (layer F.Cu) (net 4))
 (segment (start 84.795002 61.935002) (end 85.645001 62.785001) (width 0.25) (layer B.Cu) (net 5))
 (segment (start 84.47 56.595) (end 84.47 61.61) (width 0.25) (layer B.Cu) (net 5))
 (segment (start 97.67916 55.68297) (end 85.38203 55.68297) (width 0.25) (layer B.Cu) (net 5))
 (segment (start 100.56901 58.57282) (end 97.67916 55.68297) (width 0.25) (layer B.Cu) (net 5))
 (segment (start 85.38203 55.68297) (end 84.47 56.595) (width 0.25) (layer B.Cu) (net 5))
 (segment (start 100.56901 63.71949) (end 100.56901 58.57282) (width 0.25) (layer B.Cu) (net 5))
 (segment (start 100.2805 64.008) (end 100.56901 63.71949) (width 0.25) (layer B.Cu) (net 5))
 (segment (start 84.47 61.61) (end 84.795002 61.935002) (width 0.25) (layer B.Cu) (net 5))
 (segment (start 99.568 64.008) (end 100.2805 64.008) (width 0.25) (layer B.Cu) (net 5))
 (segment (start 84.795002 63.635) (end 85.645001 62.785001) (width 0.25) (layer F.Cu) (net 5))
 (segment (start 84.019991 64.410011) (end 84.795002 63.635) (width 0.25) (layer F.Cu) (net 5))
 (segment (start 85.081 69.040002) (end 84.019991 67.978993) (width 0.25) (layer F.Cu) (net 5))
 (segment (start 103.244998 69.040002) (end 85.081 69.040002) (width 0.25) (layer F.Cu) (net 5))
 (segment (start 84.019991 67.978993) (end 84.019991 64.410011) (width 0.25) (layer F.Cu) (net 5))
 (segment (start 107.205 65.08) (end 103.244998 69.040002) (width 0.25) (layer F.Cu) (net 5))
 (segment (start 107.205 64.505) (end 107.205 65.08) (width 0.25) (layer F.Cu) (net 5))
 (segment (start 86.495 59.395002) (end 85.645001 60.245001) (width 0.25) (layer B.Cu) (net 6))
 (segment (start 86.495 59.34081) (end 86.495 59.395002) (width 0.25) (layer B.Cu) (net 6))
 (segment (start 95.51598 56.13298) (end 89.70283 56.13298) (width 0.25) (layer B.Cu) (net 6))
 (segment (start 89.70283 56.13298) (end 86.495 59.34081) (width 0.25) (layer B.Cu) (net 6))
 (segment (start 98.819 59.436) (end 95.51598 56.13298) (width 0.25) (layer B.Cu) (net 6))
 (segment (start 99.5315 59.436) (end 98.819 59.436) (width 0.25) (layer B.Cu) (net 6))
 (segment (start 86.847082 60.245001) (end 85.645001 60.245001) (width 0.25) (layer F.Cu) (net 6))
 (segment (start 108.955001 61.909999) (end 107.290003 60.245001) (width 0.25) (layer F.Cu) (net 6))
 (segment (start 107.290003 60.245001) (end 86.847082 60.245001) (width 0.25) (layer F.Cu) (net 6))
 (segment (start 108.255 63.93) (end 108.955001 63.229999) (width 0.25) (layer F.Cu) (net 6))
 (segment (start 108.955001 63.229999) (end 108.955001 61.909999) (width 0.25) (layer F.Cu) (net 6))
 (segment (start 108.255 64.505) (end 108.255 63.93) (width 0.25) (layer F.Cu) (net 6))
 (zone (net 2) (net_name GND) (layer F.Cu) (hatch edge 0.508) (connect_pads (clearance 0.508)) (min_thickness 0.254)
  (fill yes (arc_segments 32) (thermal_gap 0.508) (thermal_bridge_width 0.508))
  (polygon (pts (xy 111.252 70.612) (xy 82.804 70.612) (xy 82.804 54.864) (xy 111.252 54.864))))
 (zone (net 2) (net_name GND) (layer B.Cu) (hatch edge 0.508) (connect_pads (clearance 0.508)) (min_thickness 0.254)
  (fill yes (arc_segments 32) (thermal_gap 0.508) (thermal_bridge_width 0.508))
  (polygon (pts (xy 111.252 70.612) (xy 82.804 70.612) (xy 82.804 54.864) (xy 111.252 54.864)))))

